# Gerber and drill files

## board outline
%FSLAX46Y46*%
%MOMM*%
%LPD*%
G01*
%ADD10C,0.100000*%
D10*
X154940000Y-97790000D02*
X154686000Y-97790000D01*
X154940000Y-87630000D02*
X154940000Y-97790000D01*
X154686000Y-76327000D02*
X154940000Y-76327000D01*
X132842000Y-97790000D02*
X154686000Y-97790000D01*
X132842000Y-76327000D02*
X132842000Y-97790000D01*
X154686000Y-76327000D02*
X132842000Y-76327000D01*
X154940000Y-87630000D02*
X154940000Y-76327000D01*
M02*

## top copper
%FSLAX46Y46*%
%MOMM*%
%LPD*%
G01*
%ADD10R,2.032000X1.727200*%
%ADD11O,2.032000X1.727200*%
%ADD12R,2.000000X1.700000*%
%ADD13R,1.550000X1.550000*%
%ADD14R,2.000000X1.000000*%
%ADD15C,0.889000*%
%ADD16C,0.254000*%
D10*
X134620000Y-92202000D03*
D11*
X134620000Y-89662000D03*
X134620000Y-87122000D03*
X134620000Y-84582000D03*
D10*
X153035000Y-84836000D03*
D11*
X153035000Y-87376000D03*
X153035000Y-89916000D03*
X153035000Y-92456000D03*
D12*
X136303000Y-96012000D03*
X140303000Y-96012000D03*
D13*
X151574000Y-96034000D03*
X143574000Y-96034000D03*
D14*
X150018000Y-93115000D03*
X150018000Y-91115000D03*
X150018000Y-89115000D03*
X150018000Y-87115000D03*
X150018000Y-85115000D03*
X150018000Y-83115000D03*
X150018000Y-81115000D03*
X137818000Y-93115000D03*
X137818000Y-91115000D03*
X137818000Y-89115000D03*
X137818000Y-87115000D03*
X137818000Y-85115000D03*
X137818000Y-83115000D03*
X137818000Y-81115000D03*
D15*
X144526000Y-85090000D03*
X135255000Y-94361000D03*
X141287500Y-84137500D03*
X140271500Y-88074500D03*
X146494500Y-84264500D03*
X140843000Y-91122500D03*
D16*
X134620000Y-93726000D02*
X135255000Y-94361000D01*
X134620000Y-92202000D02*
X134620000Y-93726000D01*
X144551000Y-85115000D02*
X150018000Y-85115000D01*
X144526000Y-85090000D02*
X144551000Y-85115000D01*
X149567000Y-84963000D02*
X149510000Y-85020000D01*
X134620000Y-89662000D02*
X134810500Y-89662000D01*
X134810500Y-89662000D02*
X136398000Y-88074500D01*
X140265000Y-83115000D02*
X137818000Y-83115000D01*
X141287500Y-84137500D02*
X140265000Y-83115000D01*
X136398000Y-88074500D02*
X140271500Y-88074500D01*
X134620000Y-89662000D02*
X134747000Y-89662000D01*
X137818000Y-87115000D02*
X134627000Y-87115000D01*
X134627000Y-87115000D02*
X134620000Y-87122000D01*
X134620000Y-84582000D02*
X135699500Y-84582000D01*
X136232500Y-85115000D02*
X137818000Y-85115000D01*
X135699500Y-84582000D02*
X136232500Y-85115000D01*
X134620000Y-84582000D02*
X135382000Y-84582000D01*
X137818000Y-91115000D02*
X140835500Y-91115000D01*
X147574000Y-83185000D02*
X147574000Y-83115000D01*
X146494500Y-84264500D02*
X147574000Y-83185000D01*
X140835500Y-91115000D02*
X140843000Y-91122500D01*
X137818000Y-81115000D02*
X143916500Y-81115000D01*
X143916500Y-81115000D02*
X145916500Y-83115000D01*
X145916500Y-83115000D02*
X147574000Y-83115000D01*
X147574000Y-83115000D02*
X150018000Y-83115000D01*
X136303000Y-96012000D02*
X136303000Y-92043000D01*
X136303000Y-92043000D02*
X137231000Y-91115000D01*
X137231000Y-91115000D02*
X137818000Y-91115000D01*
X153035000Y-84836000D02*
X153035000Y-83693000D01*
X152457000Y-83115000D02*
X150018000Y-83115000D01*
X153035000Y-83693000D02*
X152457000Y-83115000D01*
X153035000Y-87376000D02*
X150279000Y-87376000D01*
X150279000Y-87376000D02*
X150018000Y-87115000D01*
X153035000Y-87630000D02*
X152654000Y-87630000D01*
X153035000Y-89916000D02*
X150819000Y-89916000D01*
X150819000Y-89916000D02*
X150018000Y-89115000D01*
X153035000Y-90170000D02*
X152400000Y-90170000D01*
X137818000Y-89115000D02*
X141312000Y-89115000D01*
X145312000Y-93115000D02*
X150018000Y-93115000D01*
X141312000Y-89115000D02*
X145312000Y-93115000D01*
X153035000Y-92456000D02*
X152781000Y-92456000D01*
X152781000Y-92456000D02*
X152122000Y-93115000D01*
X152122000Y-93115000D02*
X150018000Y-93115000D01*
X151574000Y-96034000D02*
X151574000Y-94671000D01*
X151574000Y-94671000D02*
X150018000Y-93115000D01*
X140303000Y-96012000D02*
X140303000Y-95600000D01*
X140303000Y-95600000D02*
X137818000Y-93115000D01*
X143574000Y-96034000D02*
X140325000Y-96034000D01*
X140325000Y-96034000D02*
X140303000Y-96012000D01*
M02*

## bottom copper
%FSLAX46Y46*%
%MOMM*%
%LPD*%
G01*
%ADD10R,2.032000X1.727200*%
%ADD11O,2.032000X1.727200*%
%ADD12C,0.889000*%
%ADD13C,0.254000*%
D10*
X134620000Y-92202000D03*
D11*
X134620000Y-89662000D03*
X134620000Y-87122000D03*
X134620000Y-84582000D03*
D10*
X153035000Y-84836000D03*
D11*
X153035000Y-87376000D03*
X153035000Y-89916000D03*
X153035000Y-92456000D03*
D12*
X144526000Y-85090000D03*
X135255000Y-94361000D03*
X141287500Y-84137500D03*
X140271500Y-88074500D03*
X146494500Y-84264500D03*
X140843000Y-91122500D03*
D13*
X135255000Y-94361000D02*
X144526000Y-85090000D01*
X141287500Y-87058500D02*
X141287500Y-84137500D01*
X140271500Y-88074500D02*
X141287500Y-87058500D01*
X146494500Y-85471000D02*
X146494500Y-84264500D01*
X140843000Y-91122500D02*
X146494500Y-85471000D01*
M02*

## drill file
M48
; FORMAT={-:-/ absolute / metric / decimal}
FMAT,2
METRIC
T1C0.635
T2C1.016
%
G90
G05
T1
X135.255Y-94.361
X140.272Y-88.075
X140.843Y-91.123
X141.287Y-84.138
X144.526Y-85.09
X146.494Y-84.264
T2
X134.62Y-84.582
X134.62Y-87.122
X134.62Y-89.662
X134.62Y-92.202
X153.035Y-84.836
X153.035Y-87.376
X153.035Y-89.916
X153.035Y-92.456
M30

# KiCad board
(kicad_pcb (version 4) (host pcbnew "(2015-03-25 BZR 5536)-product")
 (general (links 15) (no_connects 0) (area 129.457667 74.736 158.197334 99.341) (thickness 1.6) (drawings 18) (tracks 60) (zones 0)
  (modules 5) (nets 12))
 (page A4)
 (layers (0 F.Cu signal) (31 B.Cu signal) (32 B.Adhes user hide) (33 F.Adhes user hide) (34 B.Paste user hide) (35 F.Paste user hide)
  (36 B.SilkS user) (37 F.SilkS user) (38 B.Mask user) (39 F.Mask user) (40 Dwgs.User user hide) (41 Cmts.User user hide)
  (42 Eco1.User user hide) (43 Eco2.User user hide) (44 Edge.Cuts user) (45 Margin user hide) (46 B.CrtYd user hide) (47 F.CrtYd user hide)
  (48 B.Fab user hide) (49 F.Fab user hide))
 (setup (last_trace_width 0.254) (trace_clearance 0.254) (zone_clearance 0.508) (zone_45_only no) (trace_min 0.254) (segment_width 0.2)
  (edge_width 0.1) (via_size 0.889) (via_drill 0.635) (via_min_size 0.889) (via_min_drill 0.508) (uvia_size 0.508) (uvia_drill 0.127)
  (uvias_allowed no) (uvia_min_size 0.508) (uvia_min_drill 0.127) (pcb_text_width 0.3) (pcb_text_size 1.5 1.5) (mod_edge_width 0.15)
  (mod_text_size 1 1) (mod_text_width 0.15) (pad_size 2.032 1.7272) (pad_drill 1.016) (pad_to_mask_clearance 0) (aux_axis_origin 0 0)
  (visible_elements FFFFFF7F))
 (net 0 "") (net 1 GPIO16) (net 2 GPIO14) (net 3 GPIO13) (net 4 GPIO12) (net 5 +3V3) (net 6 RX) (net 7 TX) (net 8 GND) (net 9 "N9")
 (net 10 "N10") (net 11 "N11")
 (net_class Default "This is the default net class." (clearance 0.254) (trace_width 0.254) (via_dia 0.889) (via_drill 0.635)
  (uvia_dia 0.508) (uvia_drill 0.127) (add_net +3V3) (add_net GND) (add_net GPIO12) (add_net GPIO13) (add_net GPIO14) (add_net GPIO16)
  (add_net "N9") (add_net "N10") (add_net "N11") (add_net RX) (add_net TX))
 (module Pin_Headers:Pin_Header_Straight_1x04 (layer F.Cu) (at 134.62 92.202 180)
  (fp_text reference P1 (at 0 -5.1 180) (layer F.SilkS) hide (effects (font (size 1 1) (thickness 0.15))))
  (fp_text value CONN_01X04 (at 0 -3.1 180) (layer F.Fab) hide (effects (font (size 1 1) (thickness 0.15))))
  (pad 1 thru_hole rect (at 0 0 180) (size 2.032 1.7272) (drill 1.016) (layers *.Cu *.Mask F.SilkS) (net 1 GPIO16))
  (pad 2 thru_hole oval (at 0 2.54 180) (size 2.032 1.7272) (drill 1.016) (layers *.Cu *.Mask F.SilkS) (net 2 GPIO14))
  (pad 3 thru_hole oval (at 0 5.08 180) (size 2.032 1.7272) (drill 1.016) (layers *.Cu *.Mask F.SilkS) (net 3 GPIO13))
  (pad 4 thru_hole oval (at 0 7.62 180) (size 2.032 1.7272) (drill 1.016) (layers *.Cu *.Mask F.SilkS) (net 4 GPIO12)))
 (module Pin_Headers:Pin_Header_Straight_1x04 (layer F.Cu) (at 153.035 84.836)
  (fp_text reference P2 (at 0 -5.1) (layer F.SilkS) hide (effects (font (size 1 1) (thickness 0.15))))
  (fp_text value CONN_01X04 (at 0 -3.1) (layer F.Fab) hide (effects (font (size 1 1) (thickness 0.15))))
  (pad 1 thru_hole rect (at 0 0) (size 2.032 1.7272) (drill 1.016) (layers *.Cu *.Mask F.SilkS) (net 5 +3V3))
  (pad 2 thru_hole oval (at 0 2.54) (size 2.032 1.7272) (drill 1.016) (layers *.Cu *.Mask F.SilkS) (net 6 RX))
  (pad 3 thru_hole oval (at 0 5.08) (size 2.032 1.7272) (drill 1.016) (layers *.Cu *.Mask F.SilkS) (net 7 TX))
  (pad 4 thru_hole oval (at 0 7.62) (size 2.032 1.7272) (drill 1.016) (layers *.Cu *.Mask F.SilkS) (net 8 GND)))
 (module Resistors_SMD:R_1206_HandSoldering (layer F.Cu) (at 138.303 96.012)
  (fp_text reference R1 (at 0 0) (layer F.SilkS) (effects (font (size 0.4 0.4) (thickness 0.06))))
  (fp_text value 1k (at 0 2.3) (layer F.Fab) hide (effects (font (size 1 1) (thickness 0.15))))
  (pad 1 smd rect (at -2 0) (size 2 1.7) (layers F.Cu F.Paste F.Mask) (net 5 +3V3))
  (pad 2 smd rect (at 2 0) (size 2 1.7) (layers F.Cu F.Paste F.Mask) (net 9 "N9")))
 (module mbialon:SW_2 (layer F.Cu) (at 147.574 94.234 180)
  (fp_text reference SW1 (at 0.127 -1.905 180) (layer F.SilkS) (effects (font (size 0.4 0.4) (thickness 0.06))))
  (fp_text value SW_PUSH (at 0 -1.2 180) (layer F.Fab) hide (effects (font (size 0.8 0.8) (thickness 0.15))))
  (pad 1 smd rect (at -4 -1.8 180) (size 1.55 1.55) (layers F.Cu F.Paste F.Mask) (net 8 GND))
  (pad 2 smd rect (at 4 -1.8 180) (size 1.55 1.55) (layers F.Cu F.Paste F.Mask) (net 9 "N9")))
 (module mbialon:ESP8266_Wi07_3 (layer F.Cu) (at 144.018 81.915)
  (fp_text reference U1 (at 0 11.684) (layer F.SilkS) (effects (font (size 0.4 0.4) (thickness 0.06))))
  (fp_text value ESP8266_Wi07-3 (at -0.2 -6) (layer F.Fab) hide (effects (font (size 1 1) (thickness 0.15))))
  (pad 1 smd rect (at 6 11.2) (size 2 1) (layers F.Cu F.Paste F.Mask) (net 8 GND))
  (pad 2 smd rect (at 6 9.2) (size 2 1) (layers F.Cu F.Paste F.Mask) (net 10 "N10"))
  (pad 3 smd rect (at 6 7.2) (size 2 1) (layers F.Cu F.Paste F.Mask) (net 7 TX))
  (pad 4 smd rect (at 6 5.2) (size 2 1) (layers F.Cu F.Paste F.Mask) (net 6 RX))
  (pad 5 smd rect (at 6 3.2) (size 2 1) (layers F.Cu F.Paste F.Mask) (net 1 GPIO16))
  (pad 6 smd rect (at 6 1.2) (size 2 1) (layers F.Cu F.Paste F.Mask) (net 5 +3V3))
  (pad 7 smd rect (at 6 -0.8) (size 2 1) (layers F.Cu F.Paste F.Mask) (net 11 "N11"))
  (pad 14 smd rect (at -6.2 11.2) (size 2 1) (layers F.Cu F.Paste F.Mask) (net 9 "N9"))
  (pad 13 smd rect (at -6.2 9.2) (size 2 1) (layers F.Cu F.Paste F.Mask) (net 5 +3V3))
  (pad 12 smd rect (at -6.2 7.2) (size 2 1) (layers F.Cu F.Paste F.Mask) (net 8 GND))
  (pad 11 smd rect (at -6.2 5.2) (size 2 1) (layers F.Cu F.Paste F.Mask) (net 3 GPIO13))
  (pad 10 smd rect (at -6.2 3.2) (size 2 1) (layers F.Cu F.Paste F.Mask) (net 4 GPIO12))
  (pad 9 smd rect (at -6.2 1.2) (size 2 1) (layers F.Cu F.Paste F.Mask) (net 2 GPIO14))
  (pad 8 smd rect (at -6.2 -0.8) (size 2 1) (layers F.Cu F.Paste F.Mask) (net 5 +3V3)))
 (gr_line (start 154.94 97.79) (end 154.686 97.79) (angle 90) (layer Edge.Cuts) (width 0.1))
 (gr_line (start 154.94 87.63) (end 154.94 97.79) (angle 90) (layer Edge.Cuts) (width 0.1))
 (gr_line (start 154.686 76.327) (end 154.94 76.327) (angle 90) (layer Edge.Cuts) (width 0.1))
 (gr_line (start 132.842 97.79) (end 154.686 97.79) (angle 90) (layer Edge.Cuts) (width 0.1))
 (gr_line (start 132.842 76.327) (end 132.842 97.79) (angle 90) (layer Edge.Cuts) (width 0.1))
 (gr_line (start 154.686 76.327) (end 132.842 76.327) (angle 90) (layer Edge.Cuts) (width 0.1))
 (gr_line (start 154.94 87.63) (end 154.94 76.327) (angle 90) (layer Edge.Cuts) (width 0.1))
 (via (at 144.526 85.09) (size 0.889) (layers F.Cu B.Cu) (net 1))
 (segment (start 134.62 93.726) (end 135.255 94.361) (width 0.254) (layer F.Cu) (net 1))
 (via (at 135.255 94.361) (size 0.889) (layers F.Cu B.Cu) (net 1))
 (segment (start 135.255 94.361) (end 144.526 85.09) (width 0.254) (layer B.Cu) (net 1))
 (segment (start 134.62 92.202) (end 134.62 93.726) (width 0.254) (layer F.Cu) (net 1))
 (segment (start 144.551 85.115) (end 150.018 85.115) (width 0.254) (layer F.Cu) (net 1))
 (segment (start 144.526 85.09) (end 144.551 85.115) (width 0.254) (layer F.Cu) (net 1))
 (segment (start 149.567 84.963) (end 149.51 85.02) (width 0.254) (layer F.Cu) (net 1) (status 30))
 (segment (start 134.62 89.662) (end 134.8105 89.662) (width 0.254) (layer F.Cu) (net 2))
 (segment (start 134.8105 89.662) (end 136.398 88.0745) (width 0.254) (layer F.Cu) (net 2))
 (segment (start 140.265 83.115) (end 137.818 83.115) (width 0.254) (layer F.Cu) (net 2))
 (segment (start 141.2875 84.1375) (end 140.265 83.115) (width 0.254) (layer F.Cu) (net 2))
 (via (at 141.2875 84.1375) (size 0.889) (layers F.Cu B.Cu) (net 2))
 (segment (start 141.2875 87.0585) (end 141.2875 84.1375) (width 0.254) (layer B.Cu) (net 2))
 (segment (start 140.2715 88.0745) (end 141.2875 87.0585) (width 0.254) (layer B.Cu) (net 2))
 (via (at 140.2715 88.0745) (size 0.889) (layers F.Cu B.Cu) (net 2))
 (segment (start 136.398 88.0745) (end 140.2715 88.0745) (width 0.254) (layer F.Cu) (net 2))
 (segment (start 134.62 89.662) (end 134.747 89.662) (width 0.254) (layer F.Cu) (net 2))
 (segment (start 137.818 87.115) (end 134.627 87.115) (width 0.254) (layer F.Cu) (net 3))
 (segment (start 134.627 87.115) (end 134.62 87.122) (width 0.254) (layer F.Cu) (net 3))
 (segment (start 134.62 84.582) (end 135.6995 84.582) (width 0.254) (layer F.Cu) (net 4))
 (segment (start 136.2325 85.115) (end 137.818 85.115) (width 0.254) (layer F.Cu) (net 4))
 (segment (start 135.6995 84.582) (end 136.2325 85.115) (width 0.254) (layer F.Cu) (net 4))
 (segment (start 134.62 84.582) (end 135.382 84.582) (width 0.254) (layer F.Cu) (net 4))
 (segment (start 137.818 91.115) (end 140.8355 91.115) (width 0.254) (layer F.Cu) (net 5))
 (segment (start 147.574 83.185) (end 147.574 83.115) (width 0.254) (layer F.Cu) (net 5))
 (segment (start 146.4945 84.2645) (end 147.574 83.185) (width 0.254) (layer F.Cu) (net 5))
 (via (at 146.4945 84.2645) (size 0.889) (layers F.Cu B.Cu) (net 5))
 (segment (start 146.4945 85.471) (end 146.4945 84.2645) (width 0.254) (layer B.Cu) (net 5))
 (segment (start 140.843 91.1225) (end 146.4945 85.471) (width 0.254) (layer B.Cu) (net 5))
 (via (at 140.843 91.1225) (size 0.889) (layers F.Cu B.Cu) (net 5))
 (segment (start 140.8355 91.115) (end 140.843 91.1225) (width 0.254) (layer F.Cu) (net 5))
 (segment (start 137.818 81.115) (end 143.9165 81.115) (width 0.254) (layer F.Cu) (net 5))
 (segment (start 143.9165 81.115) (end 145.9165 83.115) (width 0.254) (layer F.Cu) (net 5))
 (segment (start 145.9165 83.115) (end 147.574 83.115) (width 0.254) (layer F.Cu) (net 5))
 (segment (start 147.574 83.115) (end 150.018 83.115) (width 0.254) (layer F.Cu) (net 5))
 (segment (start 136.303 96.012) (end 136.303 92.043) (width 0.254) (layer F.Cu) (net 5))
 (segment (start 136.303 92.043) (end 137.231 91.115) (width 0.254) (layer F.Cu) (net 5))
 (segment (start 137.231 91.115) (end 137.818 91.115) (width 0.254) (layer F.Cu) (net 5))
 (segment (start 153.035 84.836) (end 153.035 83.693) (width 0.254) (layer F.Cu) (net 5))
 (segment (start 152.457 83.115) (end 150.018 83.115) (width 0.254) (layer F.Cu) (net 5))
 (segment (start 153.035 83.693) (end 152.457 83.115) (width 0.254) (layer F.Cu) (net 5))
 (segment (start 153.035 87.376) (end 150.279 87.376) (width 0.254) (layer F.Cu) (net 6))
 (segment (start 150.279 87.376) (end 150.018 87.115) (width 0.254) (layer F.Cu) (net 6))
 (segment (start 153.035 87.63) (end 152.654 87.63) (width 0.254) (layer F.Cu) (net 6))
 (segment (start 153.035 89.916) (end 150.819 89.916) (width 0.254) (layer F.Cu) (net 7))
 (segment (start 150.819 89.916) (end 150.018 89.115) (width 0.254) (layer F.Cu) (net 7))
 (segment (start 153.035 90.17) (end 152.4 90.17) (width 0.254) (layer F.Cu) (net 7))
 (segment (start 137.818 89.115) (end 141.312 89.115) (width 0.254) (layer F.Cu) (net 8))
 (segment (start 145.312 93.115) (end 150.018 93.115) (width 0.254) (layer F.Cu) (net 8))
 (segment (start 141.312 89.115) (end 145.312 93.115) (width 0.254) (layer F.Cu) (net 8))
 (segment (start 153.035 92.456) (end 152.781 92.456) (width 0.254) (layer F.Cu) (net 8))
 (segment (start 152.781 92.456) (end 152.122 93.115) (width 0.254) (layer F.Cu) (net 8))
 (segment (start 152.122 93.115) (end 150.018 93.115) (width 0.254) (layer F.Cu) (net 8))
 (segment (start 151.574 96.034) (end 151.574 94.671) (width 0.254) (layer F.Cu) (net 8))
 (segment (start 151.574 94.671) (end 150.018 93.115) (width 0.254) (layer F.Cu) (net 8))
 (segment (start 140.303 96.012) (end 140.303 95.6) (width 0.254) (layer F.Cu) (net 9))
 (segment (start 140.303 95.6) (end 137.818 93.115) (width 0.254) (layer F.Cu) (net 9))
 (segment (start 143.574 96.034) (end 140.325 96.034) (width 0.254) (layer F.Cu) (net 9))
 (segment (start 140.325 96.034) (end 140.303 96.012) (width 0.254) (layer F.Cu) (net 9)))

